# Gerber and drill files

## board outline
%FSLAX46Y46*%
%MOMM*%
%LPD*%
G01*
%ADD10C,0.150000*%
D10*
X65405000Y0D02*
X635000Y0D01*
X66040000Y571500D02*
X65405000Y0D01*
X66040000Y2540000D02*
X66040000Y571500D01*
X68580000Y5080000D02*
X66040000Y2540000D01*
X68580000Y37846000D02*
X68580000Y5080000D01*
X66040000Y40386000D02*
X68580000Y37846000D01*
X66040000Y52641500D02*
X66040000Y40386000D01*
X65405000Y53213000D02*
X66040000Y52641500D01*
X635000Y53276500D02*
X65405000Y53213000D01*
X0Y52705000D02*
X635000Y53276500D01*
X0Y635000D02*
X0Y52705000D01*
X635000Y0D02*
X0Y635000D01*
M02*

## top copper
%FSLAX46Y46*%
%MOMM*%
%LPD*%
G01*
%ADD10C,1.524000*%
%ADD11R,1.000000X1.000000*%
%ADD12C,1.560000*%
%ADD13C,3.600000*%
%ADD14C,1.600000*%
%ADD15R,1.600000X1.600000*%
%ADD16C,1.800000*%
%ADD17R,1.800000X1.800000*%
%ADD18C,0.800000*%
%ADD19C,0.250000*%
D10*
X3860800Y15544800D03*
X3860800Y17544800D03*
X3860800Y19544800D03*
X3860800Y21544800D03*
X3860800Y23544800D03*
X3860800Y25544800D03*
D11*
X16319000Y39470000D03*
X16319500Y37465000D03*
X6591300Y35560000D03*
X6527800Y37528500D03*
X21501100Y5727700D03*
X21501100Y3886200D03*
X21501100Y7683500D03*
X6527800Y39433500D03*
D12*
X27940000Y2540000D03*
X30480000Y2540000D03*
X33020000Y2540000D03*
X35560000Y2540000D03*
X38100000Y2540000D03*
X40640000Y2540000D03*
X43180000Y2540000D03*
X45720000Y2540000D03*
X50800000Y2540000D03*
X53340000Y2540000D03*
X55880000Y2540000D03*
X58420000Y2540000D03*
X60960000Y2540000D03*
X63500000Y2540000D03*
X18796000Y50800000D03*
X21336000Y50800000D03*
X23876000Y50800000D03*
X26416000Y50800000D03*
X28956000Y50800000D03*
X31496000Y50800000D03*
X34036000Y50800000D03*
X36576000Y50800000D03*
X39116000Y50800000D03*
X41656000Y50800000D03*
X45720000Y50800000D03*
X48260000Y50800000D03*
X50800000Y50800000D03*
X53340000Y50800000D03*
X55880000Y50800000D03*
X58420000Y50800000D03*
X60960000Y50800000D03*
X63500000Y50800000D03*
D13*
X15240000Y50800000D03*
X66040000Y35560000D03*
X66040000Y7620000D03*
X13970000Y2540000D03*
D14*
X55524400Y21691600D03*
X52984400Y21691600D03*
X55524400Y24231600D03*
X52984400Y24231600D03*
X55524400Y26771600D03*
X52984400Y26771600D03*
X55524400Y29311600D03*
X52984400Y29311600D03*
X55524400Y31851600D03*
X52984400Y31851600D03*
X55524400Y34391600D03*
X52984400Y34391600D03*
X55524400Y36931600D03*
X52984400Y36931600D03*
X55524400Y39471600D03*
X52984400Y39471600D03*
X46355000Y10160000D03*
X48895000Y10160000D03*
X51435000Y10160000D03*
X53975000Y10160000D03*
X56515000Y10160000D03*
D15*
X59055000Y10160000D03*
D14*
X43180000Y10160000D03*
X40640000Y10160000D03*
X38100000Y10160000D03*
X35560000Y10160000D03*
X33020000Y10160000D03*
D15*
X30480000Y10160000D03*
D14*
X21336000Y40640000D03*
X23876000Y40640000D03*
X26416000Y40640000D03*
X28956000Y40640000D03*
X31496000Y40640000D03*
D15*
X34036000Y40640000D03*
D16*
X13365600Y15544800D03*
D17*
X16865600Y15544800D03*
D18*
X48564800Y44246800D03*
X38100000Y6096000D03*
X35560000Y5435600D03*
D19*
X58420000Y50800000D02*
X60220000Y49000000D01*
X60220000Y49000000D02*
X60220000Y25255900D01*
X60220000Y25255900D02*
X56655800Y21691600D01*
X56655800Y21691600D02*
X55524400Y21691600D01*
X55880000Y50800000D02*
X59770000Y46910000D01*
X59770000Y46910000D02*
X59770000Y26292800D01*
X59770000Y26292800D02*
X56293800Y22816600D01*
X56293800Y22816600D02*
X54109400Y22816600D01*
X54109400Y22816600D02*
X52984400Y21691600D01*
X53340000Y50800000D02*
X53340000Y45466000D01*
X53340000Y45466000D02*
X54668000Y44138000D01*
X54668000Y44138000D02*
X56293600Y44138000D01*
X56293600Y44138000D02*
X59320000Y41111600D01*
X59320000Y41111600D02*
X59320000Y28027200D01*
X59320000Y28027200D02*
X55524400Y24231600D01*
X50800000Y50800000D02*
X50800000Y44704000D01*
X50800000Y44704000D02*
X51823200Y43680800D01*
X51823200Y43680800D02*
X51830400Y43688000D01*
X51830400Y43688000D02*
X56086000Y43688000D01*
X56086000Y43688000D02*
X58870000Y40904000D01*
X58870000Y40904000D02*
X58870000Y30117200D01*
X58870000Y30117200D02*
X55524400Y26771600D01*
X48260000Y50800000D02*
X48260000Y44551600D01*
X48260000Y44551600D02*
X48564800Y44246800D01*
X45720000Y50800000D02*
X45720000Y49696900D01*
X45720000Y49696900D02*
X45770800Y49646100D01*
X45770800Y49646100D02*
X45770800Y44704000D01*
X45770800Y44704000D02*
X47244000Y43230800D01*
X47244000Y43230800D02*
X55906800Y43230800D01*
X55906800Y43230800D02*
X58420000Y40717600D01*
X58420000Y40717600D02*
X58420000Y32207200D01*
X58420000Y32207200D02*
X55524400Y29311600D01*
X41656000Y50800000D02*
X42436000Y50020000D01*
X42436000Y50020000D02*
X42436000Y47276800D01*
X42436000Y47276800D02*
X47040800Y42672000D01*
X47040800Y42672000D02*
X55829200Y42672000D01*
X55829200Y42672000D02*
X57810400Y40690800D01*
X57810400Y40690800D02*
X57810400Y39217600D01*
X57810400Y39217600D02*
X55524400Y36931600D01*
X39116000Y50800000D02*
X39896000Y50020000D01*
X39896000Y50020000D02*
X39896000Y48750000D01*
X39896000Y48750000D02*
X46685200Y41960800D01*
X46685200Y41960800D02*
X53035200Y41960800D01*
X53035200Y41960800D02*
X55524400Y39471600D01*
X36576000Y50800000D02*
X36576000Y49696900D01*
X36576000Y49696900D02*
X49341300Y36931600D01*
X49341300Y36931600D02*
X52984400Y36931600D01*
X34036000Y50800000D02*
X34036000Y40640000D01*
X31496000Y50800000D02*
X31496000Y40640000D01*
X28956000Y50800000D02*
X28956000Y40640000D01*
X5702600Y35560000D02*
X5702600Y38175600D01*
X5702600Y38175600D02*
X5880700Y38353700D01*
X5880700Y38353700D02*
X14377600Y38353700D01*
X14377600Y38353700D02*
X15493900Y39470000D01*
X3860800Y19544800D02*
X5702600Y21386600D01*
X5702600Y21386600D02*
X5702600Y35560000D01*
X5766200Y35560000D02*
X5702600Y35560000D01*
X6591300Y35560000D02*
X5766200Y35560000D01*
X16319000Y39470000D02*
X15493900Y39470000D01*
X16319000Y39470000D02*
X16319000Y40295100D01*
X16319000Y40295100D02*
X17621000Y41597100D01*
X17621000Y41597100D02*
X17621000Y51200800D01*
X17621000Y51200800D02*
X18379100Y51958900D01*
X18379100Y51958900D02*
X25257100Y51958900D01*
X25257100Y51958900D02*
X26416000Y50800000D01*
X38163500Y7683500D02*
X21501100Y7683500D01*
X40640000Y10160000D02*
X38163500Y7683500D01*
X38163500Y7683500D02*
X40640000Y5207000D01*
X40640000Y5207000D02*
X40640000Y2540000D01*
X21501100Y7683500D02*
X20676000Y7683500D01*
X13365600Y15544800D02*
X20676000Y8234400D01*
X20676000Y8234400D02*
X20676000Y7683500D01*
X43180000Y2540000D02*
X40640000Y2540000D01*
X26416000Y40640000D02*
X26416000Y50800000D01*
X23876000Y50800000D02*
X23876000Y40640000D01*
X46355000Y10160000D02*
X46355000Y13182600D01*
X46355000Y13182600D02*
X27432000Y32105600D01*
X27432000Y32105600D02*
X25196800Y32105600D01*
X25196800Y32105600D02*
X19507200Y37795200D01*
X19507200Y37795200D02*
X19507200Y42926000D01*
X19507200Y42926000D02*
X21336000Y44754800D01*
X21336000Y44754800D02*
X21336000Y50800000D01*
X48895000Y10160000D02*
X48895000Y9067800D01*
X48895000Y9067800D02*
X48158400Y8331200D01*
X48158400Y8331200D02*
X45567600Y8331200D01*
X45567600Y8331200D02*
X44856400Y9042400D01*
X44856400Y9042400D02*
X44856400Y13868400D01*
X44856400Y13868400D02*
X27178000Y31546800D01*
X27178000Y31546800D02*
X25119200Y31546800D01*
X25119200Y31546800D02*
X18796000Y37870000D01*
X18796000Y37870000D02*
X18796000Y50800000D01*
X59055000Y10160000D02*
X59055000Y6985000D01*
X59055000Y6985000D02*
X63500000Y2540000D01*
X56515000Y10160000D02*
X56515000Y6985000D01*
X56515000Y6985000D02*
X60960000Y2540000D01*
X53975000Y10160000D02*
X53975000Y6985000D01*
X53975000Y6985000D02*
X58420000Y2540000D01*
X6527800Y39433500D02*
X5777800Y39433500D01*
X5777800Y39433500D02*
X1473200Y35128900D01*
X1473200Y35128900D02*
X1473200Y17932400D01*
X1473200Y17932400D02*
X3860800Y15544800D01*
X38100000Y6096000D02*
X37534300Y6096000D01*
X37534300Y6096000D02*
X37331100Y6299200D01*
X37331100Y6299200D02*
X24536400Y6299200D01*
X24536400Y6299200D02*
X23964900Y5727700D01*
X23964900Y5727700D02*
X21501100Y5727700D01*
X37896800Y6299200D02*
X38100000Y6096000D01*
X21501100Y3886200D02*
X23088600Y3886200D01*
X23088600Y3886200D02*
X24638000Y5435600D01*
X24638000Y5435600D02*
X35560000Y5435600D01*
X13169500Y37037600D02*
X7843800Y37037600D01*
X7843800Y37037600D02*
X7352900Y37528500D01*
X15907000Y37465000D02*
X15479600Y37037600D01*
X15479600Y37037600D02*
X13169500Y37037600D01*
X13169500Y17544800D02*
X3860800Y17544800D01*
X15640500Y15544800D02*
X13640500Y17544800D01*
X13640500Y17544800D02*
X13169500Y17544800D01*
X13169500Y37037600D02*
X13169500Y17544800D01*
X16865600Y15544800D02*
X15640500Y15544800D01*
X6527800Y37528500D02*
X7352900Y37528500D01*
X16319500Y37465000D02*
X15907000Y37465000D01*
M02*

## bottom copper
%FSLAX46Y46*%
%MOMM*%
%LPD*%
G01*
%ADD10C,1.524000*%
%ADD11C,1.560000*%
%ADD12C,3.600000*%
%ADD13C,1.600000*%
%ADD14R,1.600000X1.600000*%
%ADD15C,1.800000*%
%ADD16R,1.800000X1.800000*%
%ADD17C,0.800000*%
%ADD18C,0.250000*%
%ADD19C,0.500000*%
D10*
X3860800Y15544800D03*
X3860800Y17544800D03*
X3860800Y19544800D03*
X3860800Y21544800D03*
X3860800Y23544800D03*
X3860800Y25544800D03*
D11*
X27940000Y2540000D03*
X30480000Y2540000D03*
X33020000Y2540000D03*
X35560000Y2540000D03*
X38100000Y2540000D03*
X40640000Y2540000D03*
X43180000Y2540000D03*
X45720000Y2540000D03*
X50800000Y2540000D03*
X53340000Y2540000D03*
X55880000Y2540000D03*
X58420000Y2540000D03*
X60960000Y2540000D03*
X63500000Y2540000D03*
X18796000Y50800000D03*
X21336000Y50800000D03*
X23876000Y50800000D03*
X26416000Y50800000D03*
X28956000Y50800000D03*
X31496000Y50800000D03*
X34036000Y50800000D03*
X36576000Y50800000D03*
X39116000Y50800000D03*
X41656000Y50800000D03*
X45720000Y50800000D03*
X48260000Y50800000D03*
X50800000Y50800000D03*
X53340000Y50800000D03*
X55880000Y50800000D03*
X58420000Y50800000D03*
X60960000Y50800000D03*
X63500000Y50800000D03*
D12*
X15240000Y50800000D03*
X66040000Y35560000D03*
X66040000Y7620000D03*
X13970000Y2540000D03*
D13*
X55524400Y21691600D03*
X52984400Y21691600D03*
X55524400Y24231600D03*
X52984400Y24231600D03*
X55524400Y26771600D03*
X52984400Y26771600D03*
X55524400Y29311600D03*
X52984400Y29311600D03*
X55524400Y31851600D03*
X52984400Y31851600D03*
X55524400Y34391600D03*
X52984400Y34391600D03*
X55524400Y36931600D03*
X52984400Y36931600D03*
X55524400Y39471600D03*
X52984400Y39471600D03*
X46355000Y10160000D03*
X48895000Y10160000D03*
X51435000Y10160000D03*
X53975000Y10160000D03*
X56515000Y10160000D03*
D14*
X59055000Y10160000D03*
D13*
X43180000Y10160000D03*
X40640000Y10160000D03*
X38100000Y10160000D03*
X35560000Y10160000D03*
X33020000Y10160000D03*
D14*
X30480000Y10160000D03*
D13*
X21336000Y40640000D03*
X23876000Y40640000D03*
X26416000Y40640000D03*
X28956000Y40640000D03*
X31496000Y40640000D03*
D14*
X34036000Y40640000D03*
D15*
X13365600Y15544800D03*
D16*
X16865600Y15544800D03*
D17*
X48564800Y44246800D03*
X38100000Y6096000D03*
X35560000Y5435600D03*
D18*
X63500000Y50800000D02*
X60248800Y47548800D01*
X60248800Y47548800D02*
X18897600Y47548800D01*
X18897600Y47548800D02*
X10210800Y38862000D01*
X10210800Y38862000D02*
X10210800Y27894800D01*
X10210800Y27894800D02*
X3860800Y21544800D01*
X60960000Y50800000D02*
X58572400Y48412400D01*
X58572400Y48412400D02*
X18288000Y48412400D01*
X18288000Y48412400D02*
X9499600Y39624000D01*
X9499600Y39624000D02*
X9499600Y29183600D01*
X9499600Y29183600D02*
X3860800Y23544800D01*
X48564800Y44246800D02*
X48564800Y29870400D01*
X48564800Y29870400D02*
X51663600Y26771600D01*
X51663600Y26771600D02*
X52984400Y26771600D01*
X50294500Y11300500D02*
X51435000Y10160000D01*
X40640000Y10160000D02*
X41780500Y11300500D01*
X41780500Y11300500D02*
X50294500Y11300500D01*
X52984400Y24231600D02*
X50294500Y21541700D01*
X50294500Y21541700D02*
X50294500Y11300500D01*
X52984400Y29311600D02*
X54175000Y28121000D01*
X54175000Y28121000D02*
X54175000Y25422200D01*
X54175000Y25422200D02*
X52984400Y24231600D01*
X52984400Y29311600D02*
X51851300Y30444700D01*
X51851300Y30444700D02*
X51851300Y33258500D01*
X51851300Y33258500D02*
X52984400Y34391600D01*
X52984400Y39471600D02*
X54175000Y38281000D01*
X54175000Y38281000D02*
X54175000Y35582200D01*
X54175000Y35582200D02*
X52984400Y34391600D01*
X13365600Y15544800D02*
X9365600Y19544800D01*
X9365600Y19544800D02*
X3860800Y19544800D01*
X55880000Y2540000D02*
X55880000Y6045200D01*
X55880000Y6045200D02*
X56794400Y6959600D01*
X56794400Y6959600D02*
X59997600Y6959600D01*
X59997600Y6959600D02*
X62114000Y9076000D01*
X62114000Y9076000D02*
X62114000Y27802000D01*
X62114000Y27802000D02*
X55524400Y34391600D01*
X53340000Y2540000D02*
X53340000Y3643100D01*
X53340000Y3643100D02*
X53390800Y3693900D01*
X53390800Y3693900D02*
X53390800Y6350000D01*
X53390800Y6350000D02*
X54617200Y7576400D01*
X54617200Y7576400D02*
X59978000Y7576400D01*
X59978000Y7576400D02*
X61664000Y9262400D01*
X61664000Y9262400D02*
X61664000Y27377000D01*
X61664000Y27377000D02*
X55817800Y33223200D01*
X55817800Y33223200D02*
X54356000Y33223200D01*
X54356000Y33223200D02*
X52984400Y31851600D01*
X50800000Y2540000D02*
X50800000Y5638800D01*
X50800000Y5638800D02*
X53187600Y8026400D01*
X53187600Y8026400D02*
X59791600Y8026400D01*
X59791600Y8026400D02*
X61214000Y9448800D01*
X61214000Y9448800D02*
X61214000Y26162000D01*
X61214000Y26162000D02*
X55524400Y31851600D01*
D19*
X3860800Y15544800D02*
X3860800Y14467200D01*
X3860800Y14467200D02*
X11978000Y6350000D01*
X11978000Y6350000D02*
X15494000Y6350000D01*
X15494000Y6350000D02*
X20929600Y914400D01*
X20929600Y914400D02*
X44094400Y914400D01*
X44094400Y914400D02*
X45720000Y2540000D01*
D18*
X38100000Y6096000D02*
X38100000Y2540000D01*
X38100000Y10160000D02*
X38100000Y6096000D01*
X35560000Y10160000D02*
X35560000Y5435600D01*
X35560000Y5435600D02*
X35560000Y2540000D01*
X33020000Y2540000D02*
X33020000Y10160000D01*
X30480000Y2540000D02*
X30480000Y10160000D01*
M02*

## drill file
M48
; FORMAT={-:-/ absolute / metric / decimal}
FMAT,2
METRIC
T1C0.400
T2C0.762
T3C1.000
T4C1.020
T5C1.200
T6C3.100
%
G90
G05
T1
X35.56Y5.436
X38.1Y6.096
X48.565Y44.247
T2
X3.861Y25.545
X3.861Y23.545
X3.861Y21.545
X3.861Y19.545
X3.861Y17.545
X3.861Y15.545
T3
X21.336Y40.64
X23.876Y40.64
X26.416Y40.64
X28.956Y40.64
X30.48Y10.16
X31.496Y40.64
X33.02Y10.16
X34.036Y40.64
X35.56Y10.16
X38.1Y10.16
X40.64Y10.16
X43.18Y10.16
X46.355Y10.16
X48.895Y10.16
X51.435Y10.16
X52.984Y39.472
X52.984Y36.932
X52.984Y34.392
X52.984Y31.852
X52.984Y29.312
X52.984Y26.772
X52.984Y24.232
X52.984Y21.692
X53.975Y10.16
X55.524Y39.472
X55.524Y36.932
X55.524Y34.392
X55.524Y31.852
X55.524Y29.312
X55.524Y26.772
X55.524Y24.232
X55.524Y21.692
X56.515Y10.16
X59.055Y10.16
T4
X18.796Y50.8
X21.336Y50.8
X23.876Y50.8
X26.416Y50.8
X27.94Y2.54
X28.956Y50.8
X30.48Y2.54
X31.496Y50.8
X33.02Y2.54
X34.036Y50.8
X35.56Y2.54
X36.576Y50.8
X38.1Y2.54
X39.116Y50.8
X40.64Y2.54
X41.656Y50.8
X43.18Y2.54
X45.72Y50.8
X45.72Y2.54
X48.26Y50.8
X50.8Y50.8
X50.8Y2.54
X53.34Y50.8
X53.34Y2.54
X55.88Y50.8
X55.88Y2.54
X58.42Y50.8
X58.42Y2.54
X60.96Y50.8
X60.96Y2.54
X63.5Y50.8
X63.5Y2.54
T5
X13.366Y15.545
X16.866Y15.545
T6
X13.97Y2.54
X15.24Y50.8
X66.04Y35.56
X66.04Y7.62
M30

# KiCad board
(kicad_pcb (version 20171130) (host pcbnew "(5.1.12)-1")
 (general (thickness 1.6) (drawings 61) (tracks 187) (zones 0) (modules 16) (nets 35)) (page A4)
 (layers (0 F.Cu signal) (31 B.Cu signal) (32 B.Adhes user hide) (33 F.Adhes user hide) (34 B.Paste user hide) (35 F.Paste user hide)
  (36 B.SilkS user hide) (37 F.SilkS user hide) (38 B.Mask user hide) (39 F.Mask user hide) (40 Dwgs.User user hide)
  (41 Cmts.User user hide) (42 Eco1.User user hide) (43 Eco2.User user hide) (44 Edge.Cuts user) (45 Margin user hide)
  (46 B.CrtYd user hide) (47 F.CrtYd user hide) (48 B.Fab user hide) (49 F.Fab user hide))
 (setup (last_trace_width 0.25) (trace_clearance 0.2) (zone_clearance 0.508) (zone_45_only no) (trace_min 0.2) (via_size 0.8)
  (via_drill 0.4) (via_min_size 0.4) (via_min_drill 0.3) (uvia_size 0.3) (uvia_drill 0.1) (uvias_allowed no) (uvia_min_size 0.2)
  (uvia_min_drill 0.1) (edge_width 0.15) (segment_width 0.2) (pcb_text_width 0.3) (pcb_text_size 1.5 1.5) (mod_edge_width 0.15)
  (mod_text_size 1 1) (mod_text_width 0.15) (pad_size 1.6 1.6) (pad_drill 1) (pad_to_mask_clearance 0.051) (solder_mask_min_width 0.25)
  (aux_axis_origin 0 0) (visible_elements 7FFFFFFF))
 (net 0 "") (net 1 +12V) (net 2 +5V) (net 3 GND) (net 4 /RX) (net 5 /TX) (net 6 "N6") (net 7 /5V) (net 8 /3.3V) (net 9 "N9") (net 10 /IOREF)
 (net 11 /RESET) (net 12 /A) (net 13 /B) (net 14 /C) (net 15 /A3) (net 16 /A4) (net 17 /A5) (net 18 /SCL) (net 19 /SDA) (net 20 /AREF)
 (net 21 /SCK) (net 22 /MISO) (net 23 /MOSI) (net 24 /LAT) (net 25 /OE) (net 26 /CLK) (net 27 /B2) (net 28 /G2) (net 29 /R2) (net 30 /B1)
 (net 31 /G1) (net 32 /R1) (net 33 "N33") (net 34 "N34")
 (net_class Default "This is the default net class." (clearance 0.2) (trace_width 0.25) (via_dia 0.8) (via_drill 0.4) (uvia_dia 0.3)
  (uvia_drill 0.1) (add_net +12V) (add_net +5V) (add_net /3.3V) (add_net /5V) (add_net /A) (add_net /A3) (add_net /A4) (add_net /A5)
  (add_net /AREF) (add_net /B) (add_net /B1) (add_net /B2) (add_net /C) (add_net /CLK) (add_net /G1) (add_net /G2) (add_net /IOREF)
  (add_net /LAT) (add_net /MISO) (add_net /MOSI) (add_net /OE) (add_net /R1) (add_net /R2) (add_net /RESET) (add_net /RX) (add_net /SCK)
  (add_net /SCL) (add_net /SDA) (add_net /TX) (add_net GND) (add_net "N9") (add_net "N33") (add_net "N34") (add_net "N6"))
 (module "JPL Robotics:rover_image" (layer F.Cu) (at 38.4556 -27.7368 90)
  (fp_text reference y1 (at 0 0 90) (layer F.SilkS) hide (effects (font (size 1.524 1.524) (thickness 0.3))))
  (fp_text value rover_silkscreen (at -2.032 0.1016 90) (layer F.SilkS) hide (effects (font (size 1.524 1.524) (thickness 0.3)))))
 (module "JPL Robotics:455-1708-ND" (layer F.Cu) (at 3.8608 -15.5448 90)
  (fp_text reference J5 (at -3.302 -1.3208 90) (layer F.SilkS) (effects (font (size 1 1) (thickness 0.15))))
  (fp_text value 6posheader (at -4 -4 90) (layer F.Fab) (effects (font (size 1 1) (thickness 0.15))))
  (pad 1 thru_hole circle (at 0 0 90) (size 1.524 1.524) (drill 0.762) (layers *.Cu *.Mask) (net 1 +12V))
  (pad 2 thru_hole circle (at 2 0 90) (size 1.524 1.524) (drill 0.762) (layers *.Cu *.Mask) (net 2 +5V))
  (pad 3 thru_hole circle (at 4 0 90) (size 1.524 1.524) (drill 0.762) (layers *.Cu *.Mask) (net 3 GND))
  (pad 4 thru_hole circle (at 6 0 90) (size 1.524 1.524) (drill 0.762) (layers *.Cu *.Mask) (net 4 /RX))
  (pad 5 thru_hole circle (at 8 0 90) (size 1.524 1.524) (drill 0.762) (layers *.Cu *.Mask) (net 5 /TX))
  (pad 6 thru_hole circle (at 10 0 90) (size 1.524 1.524) (drill 0.762) (layers *.Cu *.Mask) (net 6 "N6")))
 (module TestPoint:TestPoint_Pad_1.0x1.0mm (layer F.Cu) (at 16.319 -39.47)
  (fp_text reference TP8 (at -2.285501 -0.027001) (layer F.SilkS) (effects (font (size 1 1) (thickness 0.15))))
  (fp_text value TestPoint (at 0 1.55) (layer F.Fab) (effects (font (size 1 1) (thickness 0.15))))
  (pad 1 smd rect (at 0 0) (size 1 1) (layers F.Cu F.Mask) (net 3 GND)))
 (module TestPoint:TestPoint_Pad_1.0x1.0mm (layer F.Cu) (at 16.3195 -37.465)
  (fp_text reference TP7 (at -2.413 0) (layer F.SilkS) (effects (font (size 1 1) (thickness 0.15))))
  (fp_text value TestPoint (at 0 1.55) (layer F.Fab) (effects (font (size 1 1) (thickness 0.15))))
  (pad 1 smd rect (at 0 0) (size 1 1) (layers F.Cu F.Mask) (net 2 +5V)))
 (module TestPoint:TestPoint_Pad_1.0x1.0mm (layer F.Cu) (at 6.5913 -35.56)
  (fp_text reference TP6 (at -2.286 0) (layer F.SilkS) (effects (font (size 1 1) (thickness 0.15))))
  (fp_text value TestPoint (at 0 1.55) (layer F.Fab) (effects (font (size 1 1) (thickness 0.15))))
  (pad 1 smd rect (at 0 0) (size 1 1) (layers F.Cu F.Mask) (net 3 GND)))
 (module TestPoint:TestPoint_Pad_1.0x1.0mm (layer F.Cu) (at 6.5278 -37.5285)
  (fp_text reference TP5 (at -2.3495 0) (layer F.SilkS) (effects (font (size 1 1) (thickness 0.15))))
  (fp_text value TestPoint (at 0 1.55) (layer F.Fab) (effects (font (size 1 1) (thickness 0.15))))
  (pad 1 smd rect (at 0 0) (size 1 1) (layers F.Cu F.Mask) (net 2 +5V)))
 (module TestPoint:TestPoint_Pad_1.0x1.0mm (layer F.Cu) (at 21.5011 -5.7277 90)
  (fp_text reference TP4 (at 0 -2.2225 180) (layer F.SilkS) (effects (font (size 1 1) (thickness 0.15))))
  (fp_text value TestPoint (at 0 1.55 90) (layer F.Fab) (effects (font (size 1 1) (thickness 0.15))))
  (pad 1 smd rect (at 0 0 90) (size 1 1) (layers F.Cu F.Mask) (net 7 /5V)))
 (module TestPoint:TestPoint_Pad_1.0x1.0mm (layer F.Cu) (at 21.5011 -3.8862 90)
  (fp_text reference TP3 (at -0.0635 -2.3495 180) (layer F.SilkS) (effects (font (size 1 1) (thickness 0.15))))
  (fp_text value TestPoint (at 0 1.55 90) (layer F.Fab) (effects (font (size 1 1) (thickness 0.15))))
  (pad 1 smd rect (at 0 0 90) (size 1 1) (layers F.Cu F.Mask) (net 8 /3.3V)))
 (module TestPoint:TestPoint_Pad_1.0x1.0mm (layer F.Cu) (at 21.5011 -7.6835 90)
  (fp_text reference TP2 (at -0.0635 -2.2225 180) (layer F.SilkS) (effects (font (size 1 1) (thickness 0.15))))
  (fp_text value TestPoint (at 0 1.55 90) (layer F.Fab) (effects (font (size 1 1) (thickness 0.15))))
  (pad 1 smd rect (at 0 0 90) (size 1 1) (layers F.Cu F.Mask) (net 3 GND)))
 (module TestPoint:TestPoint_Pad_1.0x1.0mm (layer F.Cu) (at 6.5278 -39.4335)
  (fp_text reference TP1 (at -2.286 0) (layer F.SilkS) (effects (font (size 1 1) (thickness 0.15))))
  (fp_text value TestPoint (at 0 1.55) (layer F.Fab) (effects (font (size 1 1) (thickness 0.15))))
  (pad 1 smd rect (at 0 0) (size 1 1) (layers F.Cu F.Mask) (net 1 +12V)))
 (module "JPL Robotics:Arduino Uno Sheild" (layer F.Cu) (at 0 0)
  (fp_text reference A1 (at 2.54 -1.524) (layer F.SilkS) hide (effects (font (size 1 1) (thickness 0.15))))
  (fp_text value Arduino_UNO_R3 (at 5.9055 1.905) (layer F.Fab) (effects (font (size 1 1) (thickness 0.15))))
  (pad 31 thru_hole circle (at 27.94 -2.54) (size 1.56 1.56) (drill 1.02) (layers *.Cu *.Mask) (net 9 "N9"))
  (pad 20 thru_hole circle (at 30.48 -2.54) (size 1.56 1.56) (drill 1.02) (layers *.Cu *.Mask) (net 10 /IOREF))
  (pad 21 thru_hole circle (at 33.02 -2.54) (size 1.56 1.56) (drill 1.02) (layers *.Cu *.Mask) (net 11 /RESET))
  (pad 22 thru_hole circle (at 35.56 -2.54) (size 1.56 1.56) (drill 1.02) (layers *.Cu *.Mask) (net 8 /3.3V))
  (pad 23 thru_hole circle (at 38.1 -2.54) (size 1.56 1.56) (drill 1.02) (layers *.Cu *.Mask) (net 7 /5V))
  (pad 24 thru_hole circle (at 40.64 -2.54) (size 1.56 1.56) (drill 1.02) (layers *.Cu *.Mask) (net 3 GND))
  (pad 25 thru_hole circle (at 43.18 -2.54) (size 1.56 1.56) (drill 1.02) (layers *.Cu *.Mask) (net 3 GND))
  (pad 26 thru_hole circle (at 45.72 -2.54) (size 1.56 1.56) (drill 1.02) (layers *.Cu *.Mask) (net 1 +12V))
  (pad 14 thru_hole circle (at 50.8 -2.54) (size 1.56 1.56) (drill 1.02) (layers *.Cu *.Mask) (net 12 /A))
  (pad 15 thru_hole circle (at 53.34 -2.54) (size 1.56 1.56) (drill 1.02) (layers *.Cu *.Mask) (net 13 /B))
  (pad 16 thru_hole circle (at 55.88 -2.54) (size 1.56 1.56) (drill 1.02) (layers *.Cu *.Mask) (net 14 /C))
  (pad 17 thru_hole circle (at 58.42 -2.54) (size 1.56 1.56) (drill 1.02) (layers *.Cu *.Mask) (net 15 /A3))
  (pad 18 thru_hole circle (at 60.96 -2.54) (size 1.56 1.56) (drill 1.02) (layers *.Cu *.Mask) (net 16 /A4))
  (pad 19 thru_hole circle (at 63.5 -2.54) (size 1.56 1.56) (drill 1.02) (layers *.Cu *.Mask) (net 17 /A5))
  (pad 30 thru_hole circle (at 18.796 -50.8) (size 1.56 1.56) (drill 1.02) (layers *.Cu *.Mask) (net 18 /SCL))
  (pad 29 thru_hole circle (at 21.336 -50.8) (size 1.56 1.56) (drill 1.02) (layers *.Cu *.Mask) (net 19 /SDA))
  (pad 28 thru_hole circle (at 23.876 -50.8) (size 1.56 1.56) (drill 1.02) (layers *.Cu *.Mask) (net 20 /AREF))
  (pad 27 thru_hole circle (at 26.416 -50.8) (size 1.56 1.56) (drill 1.02) (layers *.Cu *.Mask) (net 3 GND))
  (pad 13 thru_hole circle (at 28.956 -50.8) (size 1.56 1.56) (drill 1.02) (layers *.Cu *.Mask) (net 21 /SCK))
  (pad 12 thru_hole circle (at 31.496 -50.8) (size 1.56 1.56) (drill 1.02) (layers *.Cu *.Mask) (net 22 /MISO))
  (pad 11 thru_hole circle (at 34.036 -50.8) (size 1.56 1.56) (drill 1.02) (layers *.Cu *.Mask) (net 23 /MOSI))
  (pad 10 thru_hole circle (at 36.576 -50.8) (size 1.56 1.56) (drill 1.02) (layers *.Cu *.Mask) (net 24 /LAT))
  (pad 9 thru_hole circle (at 39.116 -50.8) (size 1.56 1.56) (drill 1.02) (layers *.Cu *.Mask) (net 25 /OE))
  (pad 8 thru_hole circle (at 41.656 -50.8) (size 1.56 1.56) (drill 1.02) (layers *.Cu *.Mask) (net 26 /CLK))
  (pad 7 thru_hole circle (at 45.72 -50.8) (size 1.56 1.56) (drill 1.02) (layers *.Cu *.Mask) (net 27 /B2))
  (pad 6 thru_hole circle (at 48.26 -50.8) (size 1.56 1.56) (drill 1.02) (layers *.Cu *.Mask) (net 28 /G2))
  (pad 5 thru_hole circle (at 50.8 -50.8) (size 1.56 1.56) (drill 1.02) (layers *.Cu *.Mask) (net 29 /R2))
  (pad 4 thru_hole circle (at 53.34 -50.8) (size 1.56 1.56) (drill 1.02) (layers *.Cu *.Mask) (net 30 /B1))
  (pad 3 thru_hole circle (at 55.88 -50.8) (size 1.56 1.56) (drill 1.02) (layers *.Cu *.Mask) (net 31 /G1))
  (pad 2 thru_hole circle (at 58.42 -50.8) (size 1.56 1.56) (drill 1.02) (layers *.Cu *.Mask) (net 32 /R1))
  (pad 1 thru_hole circle (at 60.96 -50.8) (size 1.56 1.56) (drill 1.02) (layers *.Cu *.Mask) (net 5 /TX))
  (pad 0 thru_hole circle (at 63.5 -50.8) (size 1.56 1.56) (drill 1.02) (layers *.Cu *.Mask) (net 4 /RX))
  (pad "" np_thru_hole circle (at 15.24 -50.8) (size 3.6 3.6) (drill 3.1) (layers *.Cu *.Mask))
  (pad "" np_thru_hole circle (at 66.04 -35.56) (size 3.6 3.6) (drill 3.1) (layers *.Cu *.Mask))
  (pad "" np_thru_hole circle (at 66.04 -7.62) (size 3.6 3.6) (drill 3.1) (layers *.Cu *.Mask))
  (pad "" np_thru_hole circle (at 13.97 -2.54) (size 3.6 3.6) (drill 3.1) (layers *.Cu *.Mask)))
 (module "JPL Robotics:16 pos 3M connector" (layer F.Cu) (at 54.2544 -30.5816 90)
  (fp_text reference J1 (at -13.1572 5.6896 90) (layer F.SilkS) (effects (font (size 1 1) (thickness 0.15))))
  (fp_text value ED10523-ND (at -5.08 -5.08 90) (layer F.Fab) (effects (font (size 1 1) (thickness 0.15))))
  (pad 1 thru_hole circle (at -8.89 1.27 90) (size 1.6 1.6) (drill 1) (layers *.Cu *.Mask) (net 32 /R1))
  (pad 2 thru_hole circle (at -8.89 -1.27 90) (size 1.6 1.6) (drill 1) (layers *.Cu *.Mask) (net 31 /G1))
  (pad 3 thru_hole circle (at -6.35 1.27 90) (size 1.6 1.6) (drill 1) (layers *.Cu *.Mask) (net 30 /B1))
  (pad 4 thru_hole circle (at -6.35 -1.27 90) (size 1.6 1.6) (drill 1) (layers *.Cu *.Mask) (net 3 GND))
  (pad 5 thru_hole circle (at -3.81 1.27 90) (size 1.6 1.6) (drill 1) (layers *.Cu *.Mask) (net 29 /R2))
  (pad 6 thru_hole circle (at -3.81 -1.27 90) (size 1.6 1.6) (drill 1) (layers *.Cu *.Mask) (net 28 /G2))
  (pad 7 thru_hole circle (at -1.27 1.27 90) (size 1.6 1.6) (drill 1) (layers *.Cu *.Mask) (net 27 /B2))
  (pad 8 thru_hole circle (at -1.27 -1.27 90) (size 1.6 1.6) (drill 1) (layers *.Cu *.Mask) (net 3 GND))
  (pad 9 thru_hole circle (at 1.27 1.27 90) (size 1.6 1.6) (drill 1) (layers *.Cu *.Mask) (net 12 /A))
  (pad 10 thru_hole circle (at 1.27 -1.27 90) (size 1.6 1.6) (drill 1) (layers *.Cu *.Mask) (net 13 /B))
  (pad 11 thru_hole circle (at 3.81 1.27 90) (size 1.6 1.6) (drill 1) (layers *.Cu *.Mask) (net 14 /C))
  (pad 12 thru_hole circle (at 3.81 -1.27 90) (size 1.6 1.6) (drill 1) (layers *.Cu *.Mask) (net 3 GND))
  (pad 13 thru_hole circle (at 6.35 1.27 90) (size 1.6 1.6) (drill 1) (layers *.Cu *.Mask) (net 26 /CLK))
  (pad 14 thru_hole circle (at 6.35 -1.27 90) (size 1.6 1.6) (drill 1) (layers *.Cu *.Mask) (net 24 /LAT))
  (pad 15 thru_hole circle (at 8.89 1.27 90) (size 1.6 1.6) (drill 1) (layers *.Cu *.Mask) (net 25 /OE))
  (pad 16 thru_hole circle (at 8.89 -1.27 90) (size 1.6 1.6) (drill 1) (layers *.Cu *.Mask) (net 3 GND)))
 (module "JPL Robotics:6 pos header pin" (layer F.Cu) (at 59.055 -10.16 180)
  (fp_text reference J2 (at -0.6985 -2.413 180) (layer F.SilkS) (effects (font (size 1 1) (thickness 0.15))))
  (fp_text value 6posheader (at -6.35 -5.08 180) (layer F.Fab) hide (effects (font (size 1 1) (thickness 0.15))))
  (pad 6 thru_hole circle (at 12.7 0 180) (size 1.6 1.6) (drill 1) (layers *.Cu *.Mask) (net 19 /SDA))
  (pad 5 thru_hole circle (at 10.16 0 180) (size 1.6 1.6) (drill 1) (layers *.Cu *.Mask) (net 18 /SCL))
  (pad 4 thru_hole circle (at 7.62 0 180) (size 1.6 1.6) (drill 1) (layers *.Cu *.Mask) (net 3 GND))
  (pad 3 thru_hole circle (at 5.08 0 180) (size 1.6 1.6) (drill 1) (layers *.Cu *.Mask) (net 15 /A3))
  (pad 2 thru_hole circle (at 2.54 0 180) (size 1.6 1.6) (drill 1) (layers *.Cu *.Mask) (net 16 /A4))
  (pad 1 thru_hole rect (at 0 0 180) (size 1.6 1.6) (drill 1) (layers *.Cu *.Mask) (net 17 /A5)))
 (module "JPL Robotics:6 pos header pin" (layer F.Cu) (at 30.48 -10.16)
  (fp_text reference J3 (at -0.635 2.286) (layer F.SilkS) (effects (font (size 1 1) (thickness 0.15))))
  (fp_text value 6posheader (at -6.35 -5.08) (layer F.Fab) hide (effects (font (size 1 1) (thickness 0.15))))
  (pad 6 thru_hole circle (at 12.7 0) (size 1.6 1.6) (drill 1) (layers *.Cu *.Mask) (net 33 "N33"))
  (pad 5 thru_hole circle (at 10.16 0) (size 1.6 1.6) (drill 1) (layers *.Cu *.Mask) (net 3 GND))
  (pad 4 thru_hole circle (at 7.62 0) (size 1.6 1.6) (drill 1) (layers *.Cu *.Mask) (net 7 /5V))
  (pad 3 thru_hole circle (at 5.08 0) (size 1.6 1.6) (drill 1) (layers *.Cu *.Mask) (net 8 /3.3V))
  (pad 2 thru_hole circle (at 2.54 0) (size 1.6 1.6) (drill 1) (layers *.Cu *.Mask) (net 11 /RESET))
  (pad 1 thru_hole rect (at 0 0) (size 1.6 1.6) (drill 1) (layers *.Cu *.Mask) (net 10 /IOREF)))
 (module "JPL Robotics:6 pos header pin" (layer F.Cu) (at 34.036 -40.64 180)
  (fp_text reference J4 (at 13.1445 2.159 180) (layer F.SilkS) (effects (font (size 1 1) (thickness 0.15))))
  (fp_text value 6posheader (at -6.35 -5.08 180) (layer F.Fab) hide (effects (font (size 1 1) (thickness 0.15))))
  (pad 6 thru_hole circle (at 12.7 0 180) (size 1.6 1.6) (drill 1) (layers *.Cu *.Mask) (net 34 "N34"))
  (pad 5 thru_hole circle (at 10.16 0 180) (size 1.6 1.6) (drill 1) (layers *.Cu *.Mask) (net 20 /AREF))
  (pad 4 thru_hole circle (at 7.62 0 180) (size 1.6 1.6) (drill 1) (layers *.Cu *.Mask) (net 3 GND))
  (pad 3 thru_hole circle (at 5.08 0 180) (size 1.6 1.6) (drill 1) (layers *.Cu *.Mask) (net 21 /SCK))
  (pad 2 thru_hole circle (at 2.54 0 180) (size 1.6 1.6) (drill 1) (layers *.Cu *.Mask) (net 22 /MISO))
  (pad 1 thru_hole rect (at 0 0 180) (size 1.6 1.6) (drill 1) (layers *.Cu *.Mask) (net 23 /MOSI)))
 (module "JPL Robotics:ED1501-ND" (layer F.Cu) (at 16.8656 -15.5448 180)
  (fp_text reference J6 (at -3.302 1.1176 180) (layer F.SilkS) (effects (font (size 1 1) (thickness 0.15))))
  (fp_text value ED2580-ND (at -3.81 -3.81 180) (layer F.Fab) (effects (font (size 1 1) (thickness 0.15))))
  (pad 2 thru_hole circle (at 3.5 0 180) (size 1.8 1.8) (drill 1.2) (layers *.Cu *.Mask) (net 3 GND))
  (pad 1 thru_hole rect (at 0 0 180) (size 1.8 1.8) (drill 1.2) (layers *.Cu *.Mask) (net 2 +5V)))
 (gr_line (start 65.405 0) (end 0.635 0) (layer Edge.Cuts) (width 0.15))
 (gr_line (start 66.04 -0.5715) (end 65.405 0) (layer Edge.Cuts) (width 0.15))
 (gr_line (start 66.04 -2.54) (end 66.04 -0.5715) (layer Edge.Cuts) (width 0.15))
 (gr_line (start 68.58 -5.08) (end 66.04 -2.54) (layer Edge.Cuts) (width 0.15))
 (gr_line (start 68.58 -37.846) (end 68.58 -5.08) (layer Edge.Cuts) (width 0.15))
 (gr_line (start 66.04 -40.386) (end 68.58 -37.846) (layer Edge.Cuts) (width 0.15))
 (gr_line (start 66.04 -52.6415) (end 66.04 -40.386) (layer Edge.Cuts) (width 0.15))
 (gr_line (start 65.405 -53.213) (end 66.04 -52.6415) (layer Edge.Cuts) (width 0.15))
 (gr_line (start 0.635 -53.2765) (end 65.405 -53.213) (layer Edge.Cuts) (width 0.15))
 (gr_line (start 0 -52.705) (end 0.635 -53.2765) (layer Edge.Cuts) (width 0.15))
 (gr_line (start 0 -0.635) (end 0 -52.705) (layer Edge.Cuts) (width 0.15))
 (gr_line (start 0.635 0) (end 0 -0.635) (layer Edge.Cuts) (width 0.15))
 (segment (start 63.5 -50.8) (end 60.2488 -47.5488) (width 0.25) (layer B.Cu) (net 4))
 (segment (start 60.2488 -47.5488) (end 18.8976 -47.5488) (width 0.25) (layer B.Cu) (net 4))
 (segment (start 18.8976 -47.5488) (end 10.2108 -38.862) (width 0.25) (layer B.Cu) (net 4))
 (segment (start 10.2108 -38.862) (end 10.2108 -27.8948) (width 0.25) (layer B.Cu) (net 4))
 (segment (start 10.2108 -27.8948) (end 3.8608 -21.5448) (width 0.25) (layer B.Cu) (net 4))
 (segment (start 60.96 -50.8) (end 58.5724 -48.4124) (width 0.25) (layer B.Cu) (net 5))
 (segment (start 58.5724 -48.4124) (end 18.288 -48.4124) (width 0.25) (layer B.Cu) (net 5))
 (segment (start 18.288 -48.4124) (end 9.4996 -39.624) (width 0.25) (layer B.Cu) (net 5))
 (segment (start 9.4996 -39.624) (end 9.4996 -29.1836) (width 0.25) (layer B.Cu) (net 5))
 (segment (start 9.4996 -29.1836) (end 3.8608 -23.5448) (width 0.25) (layer B.Cu) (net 5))
 (segment (start 58.42 -50.8) (end 60.22 -49) (width 0.25) (layer F.Cu) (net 32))
 (segment (start 60.22 -49) (end 60.22 -25.2559) (width 0.25) (layer F.Cu) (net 32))
 (segment (start 60.22 -25.2559) (end 56.6558 -21.6916) (width 0.25) (layer F.Cu) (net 32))
 (segment (start 56.6558 -21.6916) (end 55.5244 -21.6916) (width 0.25) (layer F.Cu) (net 32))
 (segment (start 55.88 -50.8) (end 59.77 -46.91) (width 0.25) (layer F.Cu) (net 31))
 (segment (start 59.77 -46.91) (end 59.77 -26.2928) (width 0.25) (layer F.Cu) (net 31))
 (segment (start 59.77 -26.2928) (end 56.2938 -22.8166) (width 0.25) (layer F.Cu) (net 31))
 (segment (start 56.2938 -22.8166) (end 54.1094 -22.8166) (width 0.25) (layer F.Cu) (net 31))
 (segment (start 54.1094 -22.8166) (end 52.9844 -21.6916) (width 0.25) (layer F.Cu) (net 31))
 (segment (start 53.34 -50.8) (end 53.34 -45.466) (width 0.25) (layer F.Cu) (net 30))
 (segment (start 53.34 -45.466) (end 54.668 -44.138) (width 0.25) (layer F.Cu) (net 30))
 (segment (start 54.668 -44.138) (end 56.2936 -44.138) (width 0.25) (layer F.Cu) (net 30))
 (segment (start 56.2936 -44.138) (end 59.32 -41.1116) (width 0.25) (layer F.Cu) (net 30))
 (segment (start 59.32 -41.1116) (end 59.32 -28.0272) (width 0.25) (layer F.Cu) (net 30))
 (segment (start 59.32 -28.0272) (end 55.5244 -24.2316) (width 0.25) (layer F.Cu) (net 30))
 (segment (start 50.8 -50.8) (end 50.8 -44.704) (width 0.25) (layer F.Cu) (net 29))
 (segment (start 50.8 -44.704) (end 51.8232 -43.6808) (width 0.25) (layer F.Cu) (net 29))
 (segment (start 51.8232 -43.6808) (end 51.8304 -43.688) (width 0.25) (layer F.Cu) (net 29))
 (segment (start 51.8304 -43.688) (end 56.086 -43.688) (width 0.25) (layer F.Cu) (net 29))
 (segment (start 56.086 -43.688) (end 58.87 -40.904) (width 0.25) (layer F.Cu) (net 29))
 (segment (start 58.87 -40.904) (end 58.87 -30.1172) (width 0.25) (layer F.Cu) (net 29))
 (segment (start 58.87 -30.1172) (end 55.5244 -26.7716) (width 0.25) (layer F.Cu) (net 29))
 (segment (start 48.5648 -44.2468) (end 48.5648 -29.8704) (width 0.25) (layer B.Cu) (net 28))
 (segment (start 48.5648 -29.8704) (end 51.6636 -26.7716) (width 0.25) (layer B.Cu) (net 28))
 (segment (start 51.6636 -26.7716) (end 52.9844 -26.7716) (width 0.25) (layer B.Cu) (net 28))
 (segment (start 48.26 -50.8) (end 48.26 -44.5516) (width 0.25) (layer F.Cu) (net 28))
 (segment (start 48.26 -44.5516) (end 48.5648 -44.2468) (width 0.25) (layer F.Cu) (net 28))
 (via (at 48.5648 -44.2468) (size 0.8) (layers F.Cu B.Cu) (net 28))
 (segment (start 45.72 -50.8) (end 45.72 -49.6969) (width 0.25) (layer F.Cu) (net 27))
 (segment (start 45.72 -49.6969) (end 45.7708 -49.6461) (width 0.25) (layer F.Cu) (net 27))
 (segment (start 45.7708 -49.6461) (end 45.7708 -44.704) (width 0.25) (layer F.Cu) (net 27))
 (segment (start 45.7708 -44.704) (end 47.244 -43.2308) (width 0.25) (layer F.Cu) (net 27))
 (segment (start 47.244 -43.2308) (end 55.9068 -43.2308) (width 0.25) (layer F.Cu) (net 27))
 (segment (start 55.9068 -43.2308) (end 58.42 -40.7176) (width 0.25) (layer F.Cu) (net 27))
 (segment (start 58.42 -40.7176) (end 58.42 -32.2072) (width 0.25) (layer F.Cu) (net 27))
 (segment (start 58.42 -32.2072) (end 55.5244 -29.3116) (width 0.25) (layer F.Cu) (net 27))
 (segment (start 41.656 -50.8) (end 42.436 -50.02) (width 0.25) (layer F.Cu) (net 26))
 (segment (start 42.436 -50.02) (end 42.436 -47.2768) (width 0.25) (layer F.Cu) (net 26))
 (segment (start 42.436 -47.2768) (end 47.0408 -42.672) (width 0.25) (layer F.Cu) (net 26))
 (segment (start 47.0408 -42.672) (end 55.8292 -42.672) (width 0.25) (layer F.Cu) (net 26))
 (segment (start 55.8292 -42.672) (end 57.8104 -40.6908) (width 0.25) (layer F.Cu) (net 26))
 (segment (start 57.8104 -40.6908) (end 57.8104 -39.2176) (width 0.25) (layer F.Cu) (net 26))
 (segment (start 57.8104 -39.2176) (end 55.5244 -36.9316) (width 0.25) (layer F.Cu) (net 26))
 (segment (start 39.116 -50.8) (end 39.896 -50.02) (width 0.25) (layer F.Cu) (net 25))
 (segment (start 39.896 -50.02) (end 39.896 -48.75) (width 0.25) (layer F.Cu) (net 25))
 (segment (start 39.896 -48.75) (end 46.6852 -41.9608) (width 0.25) (layer F.Cu) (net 25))
 (segment (start 46.6852 -41.9608) (end 53.0352 -41.9608) (width 0.25) (layer F.Cu) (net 25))
 (segment (start 53.0352 -41.9608) (end 55.5244 -39.4716) (width 0.25) (layer F.Cu) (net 25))
 (segment (start 36.576 -50.8) (end 36.576 -49.6969) (width 0.25) (layer F.Cu) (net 24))
 (segment (start 36.576 -49.6969) (end 49.3413 -36.9316) (width 0.25) (layer F.Cu) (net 24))
 (segment (start 49.3413 -36.9316) (end 52.9844 -36.9316) (width 0.25) (layer F.Cu) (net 24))
 (segment (start 34.036 -50.8) (end 34.036 -40.64) (width 0.25) (layer F.Cu) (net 23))
 (segment (start 31.496 -50.8) (end 31.496 -40.64) (width 0.25) (layer F.Cu) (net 22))
 (segment (start 28.956 -50.8) (end 28.956 -40.64) (width 0.25) (layer F.Cu) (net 21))
 (segment (start 5.7026 -35.56) (end 5.7026 -38.1756) (width 0.25) (layer F.Cu) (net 3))
 (segment (start 5.7026 -38.1756) (end 5.8807 -38.3537) (width 0.25) (layer F.Cu) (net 3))
 (segment (start 5.8807 -38.3537) (end 14.3776 -38.3537) (width 0.25) (layer F.Cu) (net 3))
 (segment (start 14.3776 -38.3537) (end 15.4939 -39.47) (width 0.25) (layer F.Cu) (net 3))
 (segment (start 3.8608 -19.5448) (end 5.7026 -21.3866) (width 0.25) (layer F.Cu) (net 3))
 (segment (start 5.7026 -21.3866) (end 5.7026 -35.56) (width 0.25) (layer F.Cu) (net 3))
 (segment (start 5.7662 -35.56) (end 5.7026 -35.56) (width 0.25) (layer F.Cu) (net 3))
 (segment (start 6.5913 -35.56) (end 5.7662 -35.56) (width 0.25) (layer F.Cu) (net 3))
 (segment (start 16.319 -39.47) (end 15.4939 -39.47) (width 0.25) (layer F.Cu) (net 3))
 (segment (start 16.319 -39.47) (end 16.319 -40.2951) (width 0.25) (layer F.Cu) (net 3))
 (segment (start 16.319 -40.2951) (end 17.621 -41.5971) (width 0.25) (layer F.Cu) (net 3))
 (segment (start 17.621 -41.5971) (end 17.621 -51.2008) (width 0.25) (layer F.Cu) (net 3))
 (segment (start 17.621 -51.2008) (end 18.3791 -51.9589) (width 0.25) (layer F.Cu) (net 3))
 (segment (start 18.3791 -51.9589) (end 25.2571 -51.9589) (width 0.25) (layer F.Cu) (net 3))
 (segment (start 25.2571 -51.9589) (end 26.416 -50.8) (width 0.25) (layer F.Cu) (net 3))
 (segment (start 50.2945 -11.3005) (end 51.435 -10.16) (width 0.25) (layer B.Cu) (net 3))
 (segment (start 40.64 -10.16) (end 41.7805 -11.3005) (width 0.25) (layer B.Cu) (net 3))
 (segment (start 41.7805 -11.3005) (end 50.2945 -11.3005) (width 0.25) (layer B.Cu) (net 3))
 (segment (start 52.9844 -24.2316) (end 50.2945 -21.5417) (width 0.25) (layer B.Cu) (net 3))
 (segment (start 50.2945 -21.5417) (end 50.2945 -11.3005) (width 0.25) (layer B.Cu) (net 3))
 (segment (start 52.9844 -29.3116) (end 54.175 -28.121) (width 0.25) (layer B.Cu) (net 3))
 (segment (start 54.175 -28.121) (end 54.175 -25.4222) (width 0.25) (layer B.Cu) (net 3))
 (segment (start 54.175 -25.4222) (end 52.9844 -24.2316) (width 0.25) (layer B.Cu) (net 3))
 (segment (start 38.1635 -7.6835) (end 21.5011 -7.6835) (width 0.25) (layer F.Cu) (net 3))
 (segment (start 40.64 -10.16) (end 38.1635 -7.6835) (width 0.25) (layer F.Cu) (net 3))
 (segment (start 38.1635 -7.6835) (end 40.64 -5.207) (width 0.25) (layer F.Cu) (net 3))
 (segment (start 40.64 -5.207) (end 40.64 -2.54) (width 0.25) (layer F.Cu) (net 3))
 (segment (start 21.5011 -7.6835) (end 20.676 -7.6835) (width 0.25) (layer F.Cu) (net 3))
 (segment (start 13.3656 -15.5448) (end 20.676 -8.2344) (width 0.25) (layer F.Cu) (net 3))
 (segment (start 20.676 -8.2344) (end 20.676 -7.6835) (width 0.25) (layer F.Cu) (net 3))
 (segment (start 52.9844 -29.3116) (end 51.8513 -30.4447) (width 0.25) (layer B.Cu) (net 3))
 (segment (start 51.8513 -30.4447) (end 51.8513 -33.2585) (width 0.25) (layer B.Cu) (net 3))
 (segment (start 51.8513 -33.2585) (end 52.9844 -34.3916) (width 0.25) (layer B.Cu) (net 3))
 (segment (start 43.18 -2.54) (end 40.64 -2.54) (width 0.25) (layer F.Cu) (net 3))
 (segment (start 26.416 -40.64) (end 26.416 -50.8) (width 0.25) (layer F.Cu) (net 3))
 (segment (start 52.9844 -39.4716) (end 54.175 -38.281) (width 0.25) (layer B.Cu) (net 3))
 (segment (start 54.175 -38.281) (end 54.175 -35.5822) (width 0.25) (layer B.Cu) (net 3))
 (segment (start 54.175 -35.5822) (end 52.9844 -34.3916) (width 0.25) (layer B.Cu) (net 3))
 (segment (start 13.3656 -15.5448) (end 9.3656 -19.5448) (width 0.25) (layer B.Cu) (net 3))
 (segment (start 9.3656 -19.5448) (end 3.8608 -19.5448) (width 0.25) (layer B.Cu) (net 3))
 (segment (start 23.876 -50.8) (end 23.876 -40.64) (width 0.25) (layer F.Cu) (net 20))
 (segment (start 46.355 -10.16) (end 46.355 -13.1826) (width 0.25) (layer F.Cu) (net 19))
 (segment (start 46.355 -13.1826) (end 27.432 -32.1056) (width 0.25) (layer F.Cu) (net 19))
 (segment (start 27.432 -32.1056) (end 25.1968 -32.1056) (width 0.25) (layer F.Cu) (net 19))
 (segment (start 25.1968 -32.1056) (end 19.5072 -37.7952) (width 0.25) (layer F.Cu) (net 19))
 (segment (start 19.5072 -37.7952) (end 19.5072 -42.926) (width 0.25) (layer F.Cu) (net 19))
 (segment (start 19.5072 -42.926) (end 21.336 -44.7548) (width 0.25) (layer F.Cu) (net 19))
 (segment (start 21.336 -44.7548) (end 21.336 -50.8) (width 0.25) (layer F.Cu) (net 19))
 (segment (start 48.895 -10.16) (end 48.895 -9.0678) (width 0.25) (layer F.Cu) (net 18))
 (segment (start 48.895 -9.0678) (end 48.1584 -8.3312) (width 0.25) (layer F.Cu) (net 18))
 (segment (start 48.1584 -8.3312) (end 45.5676 -8.3312) (width 0.25) (layer F.Cu) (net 18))
 (segment (start 45.5676 -8.3312) (end 44.8564 -9.0424) (width 0.25) (layer F.Cu) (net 18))
 (segment (start 44.8564 -9.0424) (end 44.8564 -13.8684) (width 0.25) (layer F.Cu) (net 18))
 (segment (start 44.8564 -13.8684) (end 27.178 -31.5468) (width 0.25) (layer F.Cu) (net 18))
 (segment (start 27.178 -31.5468) (end 25.1192 -31.5468) (width 0.25) (layer F.Cu) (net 18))
 (segment (start 25.1192 -31.5468) (end 18.796 -37.87) (width 0.25) (layer F.Cu) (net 18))
 (segment (start 18.796 -37.87) (end 18.796 -50.8) (width 0.25) (layer F.Cu) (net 18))
 (segment (start 59.055 -10.16) (end 59.055 -6.985) (width 0.25) (layer F.Cu) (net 17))
 (segment (start 59.055 -6.985) (end 63.5 -2.54) (width 0.25) (layer F.Cu) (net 17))
 (segment (start 56.515 -10.16) (end 56.515 -6.985) (width 0.25) (layer F.Cu) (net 16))
 (segment (start 56.515 -6.985) (end 60.96 -2.54) (width 0.25) (layer F.Cu) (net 16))
 (segment (start 53.975 -10.16) (end 53.975 -6.985) (width 0.25) (layer F.Cu) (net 15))
 (segment (start 53.975 -6.985) (end 58.42 -2.54) (width 0.25) (layer F.Cu) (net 15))
 (segment (start 55.88 -2.54) (end 55.88 -6.0452) (width 0.25) (layer B.Cu) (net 14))
 (segment (start 55.88 -6.0452) (end 56.7944 -6.9596) (width 0.25) (layer B.Cu) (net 14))
 (segment (start 56.7944 -6.9596) (end 59.9976 -6.9596) (width 0.25) (layer B.Cu) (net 14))
 (segment (start 59.9976 -6.9596) (end 62.114 -9.076) (width 0.25) (layer B.Cu) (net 14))
 (segment (start 62.114 -9.076) (end 62.114 -27.802) (width 0.25) (layer B.Cu) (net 14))
 (segment (start 62.114 -27.802) (end 55.5244 -34.3916) (width 0.25) (layer B.Cu) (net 14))
 (segment (start 53.34 -2.54) (end 53.34 -3.6431) (width 0.25) (layer B.Cu) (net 13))
 (segment (start 53.34 -3.6431) (end 53.3908 -3.6939) (width 0.25) (layer B.Cu) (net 13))
 (segment (start 53.3908 -3.6939) (end 53.3908 -6.35) (width 0.25) (layer B.Cu) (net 13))
 (segment (start 53.3908 -6.35) (end 54.6172 -7.5764) (width 0.25) (layer B.Cu) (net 13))
 (segment (start 54.6172 -7.5764) (end 59.978 -7.5764) (width 0.25) (layer B.Cu) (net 13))
 (segment (start 59.978 -7.5764) (end 61.664 -9.2624) (width 0.25) (layer B.Cu) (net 13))
 (segment (start 61.664 -9.2624) (end 61.664 -27.377) (width 0.25) (layer B.Cu) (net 13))
 (segment (start 61.664 -27.377) (end 55.8178 -33.2232) (width 0.25) (layer B.Cu) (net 13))
 (segment (start 55.8178 -33.2232) (end 54.356 -33.2232) (width 0.25) (layer B.Cu) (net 13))
 (segment (start 54.356 -33.2232) (end 52.9844 -31.8516) (width 0.25) (layer B.Cu) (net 13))
 (segment (start 50.8 -2.54) (end 50.8 -5.6388) (width 0.25) (layer B.Cu) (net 12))
 (segment (start 50.8 -5.6388) (end 53.1876 -8.0264) (width 0.25) (layer B.Cu) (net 12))
 (segment (start 53.1876 -8.0264) (end 59.7916 -8.0264) (width 0.25) (layer B.Cu) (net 12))
 (segment (start 59.7916 -8.0264) (end 61.214 -9.4488) (width 0.25) (layer B.Cu) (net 12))
 (segment (start 61.214 -9.4488) (end 61.214 -26.162) (width 0.25) (layer B.Cu) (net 12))
 (segment (start 61.214 -26.162) (end 55.5244 -31.8516) (width 0.25) (layer B.Cu) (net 12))
 (segment (start 6.5278 -39.4335) (end 5.7778 -39.4335) (width 0.25) (layer F.Cu) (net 1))
 (segment (start 5.7778 -39.4335) (end 1.4732 -35.1289) (width 0.25) (layer F.Cu) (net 1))
 (segment (start 1.4732 -35.1289) (end 1.4732 -17.9324) (width 0.25) (layer F.Cu) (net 1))
 (segment (start 1.4732 -17.9324) (end 3.8608 -15.5448) (width 0.25) (layer F.Cu) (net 1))
 (segment (start 3.8608 -15.5448) (end 3.8608 -14.4672) (width 0.5) (layer B.Cu) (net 1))
 (segment (start 3.8608 -14.4672) (end 11.978 -6.35) (width 0.5) (layer B.Cu) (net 1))
 (segment (start 11.978 -6.35) (end 15.494 -6.35) (width 0.5) (layer B.Cu) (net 1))
 (segment (start 15.494 -6.35) (end 20.9296 -0.9144) (width 0.5) (layer B.Cu) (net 1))
 (segment (start 20.9296 -0.9144) (end 44.0944 -0.9144) (width 0.5) (layer B.Cu) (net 1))
 (segment (start 44.0944 -0.9144) (end 45.72 -2.54) (width 0.5) (layer B.Cu) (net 1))
 (segment (start 38.1 -6.096) (end 38.1 -2.54) (width 0.25) (layer B.Cu) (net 7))
 (segment (start 38.1 -6.096) (end 37.5343 -6.096) (width 0.25) (layer F.Cu) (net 7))
 (segment (start 37.5343 -6.096) (end 37.3311 -6.2992) (width 0.25) (layer F.Cu) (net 7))
 (segment (start 37.3311 -6.2992) (end 24.5364 -6.2992) (width 0.25) (layer F.Cu) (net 7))
 (segment (start 24.5364 -6.2992) (end 23.9649 -5.7277) (width 0.25) (layer F.Cu) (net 7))
 (segment (start 23.9649 -5.7277) (end 21.5011 -5.7277) (width 0.25) (layer F.Cu) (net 7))
 (segment (start 37.8968 -6.2992) (end 38.1 -6.096) (width 0.25) (layer F.Cu) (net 7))
 (segment (start 38.1 -10.16) (end 38.1 -6.096) (width 0.25) (layer B.Cu) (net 7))
 (via (at 38.1 -6.096) (size 0.8) (layers F.Cu B.Cu) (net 7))
 (segment (start 21.5011 -3.8862) (end 23.0886 -3.8862) (width 0.25) (layer F.Cu) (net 8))
 (segment (start 23.0886 -3.8862) (end 24.638 -5.4356) (width 0.25) (layer F.Cu) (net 8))
 (segment (start 24.638 -5.4356) (end 35.56 -5.4356) (width 0.25) (layer F.Cu) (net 8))
 (segment (start 35.56 -10.16) (end 35.56 -5.4356) (width 0.25) (layer B.Cu) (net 8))
 (segment (start 35.56 -5.4356) (end 35.56 -2.54) (width 0.25) (layer B.Cu) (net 8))
 (via (at 35.56 -5.4356) (size 0.8) (layers F.Cu B.Cu) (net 8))
 (segment (start 33.02 -2.54) (end 33.02 -10.16) (width 0.25) (layer B.Cu) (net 11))
 (segment (start 30.48 -2.54) (end 30.48 -10.16) (width 0.25) (layer B.Cu) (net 10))
 (segment (start 13.1695 -37.0376) (end 7.8438 -37.0376) (width 0.25) (layer F.Cu) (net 2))
 (segment (start 7.8438 -37.0376) (end 7.3529 -37.5285) (width 0.25) (layer F.Cu) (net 2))
 (segment (start 15.907 -37.465) (end 15.4796 -37.0376) (width 0.25) (layer F.Cu) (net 2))
 (segment (start 15.4796 -37.0376) (end 13.1695 -37.0376) (width 0.25) (layer F.Cu) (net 2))
 (segment (start 13.1695 -17.5448) (end 3.8608 -17.5448) (width 0.25) (layer F.Cu) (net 2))
 (segment (start 15.6405 -15.5448) (end 13.6405 -17.5448) (width 0.25) (layer F.Cu) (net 2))
 (segment (start 13.6405 -17.5448) (end 13.1695 -17.5448) (width 0.25) (layer F.Cu) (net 2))
 (segment (start 13.1695 -37.0376) (end 13.1695 -17.5448) (width 0.25) (layer F.Cu) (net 2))
 (segment (start 16.8656 -15.5448) (end 15.6405 -15.5448) (width 0.25) (layer F.Cu) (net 2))
 (segment (start 6.5278 -37.5285) (end 7.3529 -37.5285) (width 0.25) (layer F.Cu) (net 2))
 (segment (start 16.3195 -37.465) (end 15.907 -37.465) (width 0.25) (layer F.Cu) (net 2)))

